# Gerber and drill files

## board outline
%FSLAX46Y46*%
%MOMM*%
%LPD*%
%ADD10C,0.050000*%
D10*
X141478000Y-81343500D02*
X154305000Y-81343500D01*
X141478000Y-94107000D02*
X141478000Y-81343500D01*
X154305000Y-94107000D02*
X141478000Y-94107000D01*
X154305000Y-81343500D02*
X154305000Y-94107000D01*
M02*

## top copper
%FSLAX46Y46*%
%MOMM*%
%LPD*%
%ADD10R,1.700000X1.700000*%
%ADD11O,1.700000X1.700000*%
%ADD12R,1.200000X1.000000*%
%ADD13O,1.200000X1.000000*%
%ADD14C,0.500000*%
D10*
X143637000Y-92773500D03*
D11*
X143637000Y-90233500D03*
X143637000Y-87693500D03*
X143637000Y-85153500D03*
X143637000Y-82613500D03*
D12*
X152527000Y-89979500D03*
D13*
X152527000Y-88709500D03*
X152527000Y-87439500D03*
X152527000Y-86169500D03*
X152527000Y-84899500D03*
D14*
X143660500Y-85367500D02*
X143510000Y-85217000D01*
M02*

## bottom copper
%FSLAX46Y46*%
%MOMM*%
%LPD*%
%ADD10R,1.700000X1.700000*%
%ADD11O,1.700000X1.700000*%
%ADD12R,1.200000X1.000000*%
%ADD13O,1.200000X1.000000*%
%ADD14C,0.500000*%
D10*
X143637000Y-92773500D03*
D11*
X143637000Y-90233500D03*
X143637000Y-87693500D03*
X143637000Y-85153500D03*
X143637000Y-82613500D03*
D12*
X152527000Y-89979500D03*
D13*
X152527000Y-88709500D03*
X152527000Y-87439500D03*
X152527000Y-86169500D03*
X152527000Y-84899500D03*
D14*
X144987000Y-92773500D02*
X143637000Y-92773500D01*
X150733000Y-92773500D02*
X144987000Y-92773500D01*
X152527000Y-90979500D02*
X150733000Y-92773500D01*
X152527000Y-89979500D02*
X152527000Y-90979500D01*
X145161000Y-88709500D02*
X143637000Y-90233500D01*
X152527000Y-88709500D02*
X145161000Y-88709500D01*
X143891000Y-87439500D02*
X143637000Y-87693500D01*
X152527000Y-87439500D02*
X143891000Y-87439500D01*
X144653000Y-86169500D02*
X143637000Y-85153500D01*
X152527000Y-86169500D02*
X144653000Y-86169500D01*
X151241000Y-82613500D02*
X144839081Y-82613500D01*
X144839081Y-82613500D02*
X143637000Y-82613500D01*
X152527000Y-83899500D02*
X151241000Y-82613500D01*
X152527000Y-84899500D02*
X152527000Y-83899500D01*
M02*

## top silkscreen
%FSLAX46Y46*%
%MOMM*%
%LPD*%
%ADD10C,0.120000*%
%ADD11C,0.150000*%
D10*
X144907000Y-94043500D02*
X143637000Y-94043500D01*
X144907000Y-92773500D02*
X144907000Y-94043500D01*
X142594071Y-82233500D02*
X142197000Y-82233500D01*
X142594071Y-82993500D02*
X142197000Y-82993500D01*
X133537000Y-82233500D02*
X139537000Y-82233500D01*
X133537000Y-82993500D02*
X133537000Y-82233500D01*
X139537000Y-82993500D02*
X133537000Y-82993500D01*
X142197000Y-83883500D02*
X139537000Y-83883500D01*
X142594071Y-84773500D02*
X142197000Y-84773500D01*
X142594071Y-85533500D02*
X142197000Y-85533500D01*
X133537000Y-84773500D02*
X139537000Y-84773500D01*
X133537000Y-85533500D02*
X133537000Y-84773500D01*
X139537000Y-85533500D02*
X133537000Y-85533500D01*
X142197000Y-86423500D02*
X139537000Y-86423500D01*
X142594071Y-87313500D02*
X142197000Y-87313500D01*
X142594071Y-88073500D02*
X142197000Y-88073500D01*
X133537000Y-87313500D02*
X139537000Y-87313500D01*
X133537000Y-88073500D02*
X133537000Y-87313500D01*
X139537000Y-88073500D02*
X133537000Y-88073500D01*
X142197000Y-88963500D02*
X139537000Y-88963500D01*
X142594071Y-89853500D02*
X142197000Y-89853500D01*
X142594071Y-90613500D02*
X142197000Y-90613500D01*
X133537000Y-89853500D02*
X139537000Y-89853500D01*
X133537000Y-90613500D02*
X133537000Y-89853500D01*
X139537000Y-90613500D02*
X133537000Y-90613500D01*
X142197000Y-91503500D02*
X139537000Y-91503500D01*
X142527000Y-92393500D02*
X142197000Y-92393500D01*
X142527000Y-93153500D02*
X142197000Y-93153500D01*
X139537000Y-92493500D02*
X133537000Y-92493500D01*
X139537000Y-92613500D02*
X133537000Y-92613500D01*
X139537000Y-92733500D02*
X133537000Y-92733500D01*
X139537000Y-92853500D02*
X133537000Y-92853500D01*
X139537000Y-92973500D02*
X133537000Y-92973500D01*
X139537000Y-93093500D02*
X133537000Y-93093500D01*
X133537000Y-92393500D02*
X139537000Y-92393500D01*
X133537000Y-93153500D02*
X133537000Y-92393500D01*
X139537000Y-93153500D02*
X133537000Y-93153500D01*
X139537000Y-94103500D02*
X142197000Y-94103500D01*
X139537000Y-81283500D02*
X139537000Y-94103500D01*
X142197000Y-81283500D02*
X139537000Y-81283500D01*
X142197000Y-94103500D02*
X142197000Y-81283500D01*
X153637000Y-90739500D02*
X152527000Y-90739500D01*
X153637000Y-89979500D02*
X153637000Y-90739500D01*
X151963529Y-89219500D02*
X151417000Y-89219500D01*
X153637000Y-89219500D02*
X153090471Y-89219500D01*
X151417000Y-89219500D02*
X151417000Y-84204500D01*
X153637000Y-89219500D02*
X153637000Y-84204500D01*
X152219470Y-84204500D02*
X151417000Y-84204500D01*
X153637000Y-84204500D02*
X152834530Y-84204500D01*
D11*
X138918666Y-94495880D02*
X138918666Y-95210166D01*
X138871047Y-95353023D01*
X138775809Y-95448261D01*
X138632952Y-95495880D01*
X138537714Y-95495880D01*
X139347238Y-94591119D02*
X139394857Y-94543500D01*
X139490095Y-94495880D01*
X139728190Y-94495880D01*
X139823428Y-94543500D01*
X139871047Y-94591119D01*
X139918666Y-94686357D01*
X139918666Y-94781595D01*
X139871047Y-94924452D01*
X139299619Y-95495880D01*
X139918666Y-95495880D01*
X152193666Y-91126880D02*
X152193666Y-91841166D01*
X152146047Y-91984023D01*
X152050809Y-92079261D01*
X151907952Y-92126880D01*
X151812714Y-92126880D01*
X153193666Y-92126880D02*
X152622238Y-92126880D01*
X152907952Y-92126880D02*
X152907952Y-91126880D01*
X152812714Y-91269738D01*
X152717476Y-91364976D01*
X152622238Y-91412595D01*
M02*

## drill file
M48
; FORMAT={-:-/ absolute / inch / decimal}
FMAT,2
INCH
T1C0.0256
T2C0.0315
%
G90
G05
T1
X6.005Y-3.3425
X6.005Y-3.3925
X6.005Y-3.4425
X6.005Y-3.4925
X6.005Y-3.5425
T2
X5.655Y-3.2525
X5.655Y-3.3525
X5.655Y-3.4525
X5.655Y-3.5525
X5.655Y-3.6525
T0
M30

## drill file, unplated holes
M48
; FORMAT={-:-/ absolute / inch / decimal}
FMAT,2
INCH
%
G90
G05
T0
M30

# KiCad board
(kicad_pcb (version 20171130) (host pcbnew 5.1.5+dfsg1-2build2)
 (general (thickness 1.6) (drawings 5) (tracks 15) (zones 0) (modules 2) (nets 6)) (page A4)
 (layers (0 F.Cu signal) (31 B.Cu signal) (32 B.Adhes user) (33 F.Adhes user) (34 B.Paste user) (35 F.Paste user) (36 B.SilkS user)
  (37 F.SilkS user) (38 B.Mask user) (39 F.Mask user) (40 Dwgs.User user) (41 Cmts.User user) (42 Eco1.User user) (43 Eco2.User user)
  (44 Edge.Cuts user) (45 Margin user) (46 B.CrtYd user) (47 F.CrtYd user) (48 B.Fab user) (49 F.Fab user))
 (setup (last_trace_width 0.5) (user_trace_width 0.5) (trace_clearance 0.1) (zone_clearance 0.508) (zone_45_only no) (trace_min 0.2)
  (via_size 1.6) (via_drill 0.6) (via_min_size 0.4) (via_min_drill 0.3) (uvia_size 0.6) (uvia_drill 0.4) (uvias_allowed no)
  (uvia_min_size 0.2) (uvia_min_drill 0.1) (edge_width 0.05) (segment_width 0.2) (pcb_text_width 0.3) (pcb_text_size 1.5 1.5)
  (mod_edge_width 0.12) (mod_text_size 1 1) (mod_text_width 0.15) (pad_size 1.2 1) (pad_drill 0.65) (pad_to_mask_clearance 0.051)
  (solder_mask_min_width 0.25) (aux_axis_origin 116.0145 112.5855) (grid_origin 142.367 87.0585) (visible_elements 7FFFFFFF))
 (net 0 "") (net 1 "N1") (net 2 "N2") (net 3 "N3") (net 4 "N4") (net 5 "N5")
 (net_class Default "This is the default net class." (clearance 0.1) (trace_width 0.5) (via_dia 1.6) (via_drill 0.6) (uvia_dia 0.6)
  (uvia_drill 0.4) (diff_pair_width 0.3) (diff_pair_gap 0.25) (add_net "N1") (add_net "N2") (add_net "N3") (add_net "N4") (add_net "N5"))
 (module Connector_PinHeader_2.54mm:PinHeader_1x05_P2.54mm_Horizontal (layer F.Cu) (at 143.637 92.7735 180)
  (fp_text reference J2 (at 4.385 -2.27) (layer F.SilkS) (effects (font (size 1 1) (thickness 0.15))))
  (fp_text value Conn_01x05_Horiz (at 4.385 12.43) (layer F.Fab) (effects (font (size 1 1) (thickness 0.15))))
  (fp_line (start -1.27 -1.27) (end 0 -1.27) (layer F.SilkS) (width 0.12))
  (fp_line (start -1.27 0) (end -1.27 -1.27) (layer F.SilkS) (width 0.12))
  (fp_line (start 1.042929 10.54) (end 1.44 10.54) (layer F.SilkS) (width 0.12))
  (fp_line (start 1.042929 9.78) (end 1.44 9.78) (layer F.SilkS) (width 0.12))
  (fp_line (start 10.1 10.54) (end 4.1 10.54) (layer F.SilkS) (width 0.12))
  (fp_line (start 10.1 9.78) (end 10.1 10.54) (layer F.SilkS) (width 0.12))
  (fp_line (start 4.1 9.78) (end 10.1 9.78) (layer F.SilkS) (width 0.12))
  (fp_line (start 1.44 8.89) (end 4.1 8.89) (layer F.SilkS) (width 0.12))
  (fp_line (start 1.042929 8) (end 1.44 8) (layer F.SilkS) (width 0.12))
  (fp_line (start 1.042929 7.24) (end 1.44 7.24) (layer F.SilkS) (width 0.12))
  (fp_line (start 10.1 8) (end 4.1 8) (layer F.SilkS) (width 0.12))
  (fp_line (start 10.1 7.24) (end 10.1 8) (layer F.SilkS) (width 0.12))
  (fp_line (start 4.1 7.24) (end 10.1 7.24) (layer F.SilkS) (width 0.12))
  (fp_line (start 1.44 6.35) (end 4.1 6.35) (layer F.SilkS) (width 0.12))
  (fp_line (start 1.042929 5.46) (end 1.44 5.46) (layer F.SilkS) (width 0.12))
  (fp_line (start 1.042929 4.7) (end 1.44 4.7) (layer F.SilkS) (width 0.12))
  (fp_line (start 10.1 5.46) (end 4.1 5.46) (layer F.SilkS) (width 0.12))
  (fp_line (start 10.1 4.7) (end 10.1 5.46) (layer F.SilkS) (width 0.12))
  (fp_line (start 4.1 4.7) (end 10.1 4.7) (layer F.SilkS) (width 0.12))
  (fp_line (start 1.44 3.81) (end 4.1 3.81) (layer F.SilkS) (width 0.12))
  (fp_line (start 1.042929 2.92) (end 1.44 2.92) (layer F.SilkS) (width 0.12))
  (fp_line (start 1.042929 2.16) (end 1.44 2.16) (layer F.SilkS) (width 0.12))
  (fp_line (start 10.1 2.92) (end 4.1 2.92) (layer F.SilkS) (width 0.12))
  (fp_line (start 10.1 2.16) (end 10.1 2.92) (layer F.SilkS) (width 0.12))
  (fp_line (start 4.1 2.16) (end 10.1 2.16) (layer F.SilkS) (width 0.12))
  (fp_line (start 1.44 1.27) (end 4.1 1.27) (layer F.SilkS) (width 0.12))
  (fp_line (start 1.11 0.38) (end 1.44 0.38) (layer F.SilkS) (width 0.12))
  (fp_line (start 1.11 -0.38) (end 1.44 -0.38) (layer F.SilkS) (width 0.12))
  (fp_line (start 4.1 0.28) (end 10.1 0.28) (layer F.SilkS) (width 0.12))
  (fp_line (start 4.1 0.16) (end 10.1 0.16) (layer F.SilkS) (width 0.12))
  (fp_line (start 4.1 0.04) (end 10.1 0.04) (layer F.SilkS) (width 0.12))
  (fp_line (start 4.1 -0.08) (end 10.1 -0.08) (layer F.SilkS) (width 0.12))
  (fp_line (start 4.1 -0.2) (end 10.1 -0.2) (layer F.SilkS) (width 0.12))
  (fp_line (start 4.1 -0.32) (end 10.1 -0.32) (layer F.SilkS) (width 0.12))
  (fp_line (start 10.1 0.38) (end 4.1 0.38) (layer F.SilkS) (width 0.12))
  (fp_line (start 10.1 -0.38) (end 10.1 0.38) (layer F.SilkS) (width 0.12))
  (fp_line (start 4.1 -0.38) (end 10.1 -0.38) (layer F.SilkS) (width 0.12))
  (fp_line (start 4.1 -1.33) (end 1.44 -1.33) (layer F.SilkS) (width 0.12))
  (fp_line (start 4.1 11.49) (end 4.1 -1.33) (layer F.SilkS) (width 0.12))
  (fp_line (start 1.44 11.49) (end 4.1 11.49) (layer F.SilkS) (width 0.12))
  (fp_line (start 1.44 -1.33) (end 1.44 11.49) (layer F.SilkS) (width 0.12))
  (pad 1 thru_hole rect (at 0 0 180) (size 1.7 1.7) (drill 0.8) (layers *.Cu *.Mask) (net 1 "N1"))
  (pad 2 thru_hole oval (at 0 2.54 180) (size 1.7 1.7) (drill 0.8) (layers *.Cu *.Mask) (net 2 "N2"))
  (pad 3 thru_hole oval (at 0 5.08 180) (size 1.7 1.7) (drill 0.8) (layers *.Cu *.Mask) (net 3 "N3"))
  (pad 4 thru_hole oval (at 0 7.62 180) (size 1.7 1.7) (drill 0.8) (layers *.Cu *.Mask) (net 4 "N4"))
  (pad 5 thru_hole oval (at 0 10.16 180) (size 1.7 1.7) (drill 0.8) (layers *.Cu *.Mask) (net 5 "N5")))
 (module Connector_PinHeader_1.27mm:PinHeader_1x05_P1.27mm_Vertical (layer F.Cu) (at 152.527 89.9795 180)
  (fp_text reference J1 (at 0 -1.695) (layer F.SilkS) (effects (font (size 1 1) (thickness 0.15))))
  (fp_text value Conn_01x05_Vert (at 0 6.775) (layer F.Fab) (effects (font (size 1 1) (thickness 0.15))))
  (fp_line (start -1.11 -0.76) (end 0 -0.76) (layer F.SilkS) (width 0.12))
  (fp_line (start -1.11 0) (end -1.11 -0.76) (layer F.SilkS) (width 0.12))
  (fp_line (start 0.563471 0.76) (end 1.11 0.76) (layer F.SilkS) (width 0.12))
  (fp_line (start -1.11 0.76) (end -0.563471 0.76) (layer F.SilkS) (width 0.12))
  (fp_line (start 1.11 0.76) (end 1.11 5.775) (layer F.SilkS) (width 0.12))
  (fp_line (start -1.11 0.76) (end -1.11 5.775) (layer F.SilkS) (width 0.12))
  (fp_line (start 0.30753 5.775) (end 1.11 5.775) (layer F.SilkS) (width 0.12))
  (fp_line (start -1.11 5.775) (end -0.30753 5.775) (layer F.SilkS) (width 0.12))
  (pad 1 thru_hole rect (at 0 0 180) (size 1.2 1) (drill 0.65) (layers *.Cu *.Mask) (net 1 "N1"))
  (pad 2 thru_hole oval (at 0 1.27 180) (size 1.2 1) (drill 0.65) (layers *.Cu *.Mask) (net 2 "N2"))
  (pad 3 thru_hole oval (at 0 2.54 180) (size 1.2 1) (drill 0.65) (layers *.Cu *.Mask) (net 3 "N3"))
  (pad 4 thru_hole oval (at 0 3.81 180) (size 1.2 1) (drill 0.65) (layers *.Cu *.Mask) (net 4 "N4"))
  (pad 5 thru_hole oval (at 0 5.08 180) (size 1.2 1) (drill 0.65) (layers *.Cu *.Mask) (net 5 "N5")))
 (gr_line (start 141.478 81.3435) (end 154.305 81.3435) (layer Edge.Cuts) (width 0.05))
 (gr_line (start 141.478 94.107) (end 141.478 81.3435) (layer Edge.Cuts) (width 0.05))
 (gr_line (start 154.305 94.107) (end 141.478 94.107) (layer Edge.Cuts) (width 0.05))
 (gr_line (start 154.305 81.3435) (end 154.305 94.107) (layer Edge.Cuts) (width 0.05))
 (segment (start 144.987 92.7735) (end 143.637 92.7735) (width 0.5) (layer B.Cu) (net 1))
 (segment (start 150.733 92.7735) (end 144.987 92.7735) (width 0.5) (layer B.Cu) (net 1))
 (segment (start 152.527 90.9795) (end 150.733 92.7735) (width 0.5) (layer B.Cu) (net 1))
 (segment (start 152.527 89.9795) (end 152.527 90.9795) (width 0.5) (layer B.Cu) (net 1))
 (segment (start 145.161 88.7095) (end 143.637 90.2335) (width 0.5) (layer B.Cu) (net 2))
 (segment (start 152.527 88.7095) (end 145.161 88.7095) (width 0.5) (layer B.Cu) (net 2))
 (segment (start 143.891 87.4395) (end 143.637 87.6935) (width 0.5) (layer B.Cu) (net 3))
 (segment (start 152.527 87.4395) (end 143.891 87.4395) (width 0.5) (layer B.Cu) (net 3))
 (segment (start 143.6605 85.3675) (end 143.51 85.217) (width 0.5) (layer F.Cu) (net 4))
 (segment (start 144.653 86.1695) (end 143.637 85.1535) (width 0.5) (layer B.Cu) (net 4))
 (segment (start 152.527 86.1695) (end 144.653 86.1695) (width 0.5) (layer B.Cu) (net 4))
 (segment (start 151.241 82.6135) (end 144.839081 82.6135) (width 0.5) (layer B.Cu) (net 5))
 (segment (start 144.839081 82.6135) (end 143.637 82.6135) (width 0.5) (layer B.Cu) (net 5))
 (segment (start 152.527 83.8995) (end 151.241 82.6135) (width 0.5) (layer B.Cu) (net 5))
 (segment (start 152.527 84.8995) (end 152.527 83.8995) (width 0.5) (layer B.Cu) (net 5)))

